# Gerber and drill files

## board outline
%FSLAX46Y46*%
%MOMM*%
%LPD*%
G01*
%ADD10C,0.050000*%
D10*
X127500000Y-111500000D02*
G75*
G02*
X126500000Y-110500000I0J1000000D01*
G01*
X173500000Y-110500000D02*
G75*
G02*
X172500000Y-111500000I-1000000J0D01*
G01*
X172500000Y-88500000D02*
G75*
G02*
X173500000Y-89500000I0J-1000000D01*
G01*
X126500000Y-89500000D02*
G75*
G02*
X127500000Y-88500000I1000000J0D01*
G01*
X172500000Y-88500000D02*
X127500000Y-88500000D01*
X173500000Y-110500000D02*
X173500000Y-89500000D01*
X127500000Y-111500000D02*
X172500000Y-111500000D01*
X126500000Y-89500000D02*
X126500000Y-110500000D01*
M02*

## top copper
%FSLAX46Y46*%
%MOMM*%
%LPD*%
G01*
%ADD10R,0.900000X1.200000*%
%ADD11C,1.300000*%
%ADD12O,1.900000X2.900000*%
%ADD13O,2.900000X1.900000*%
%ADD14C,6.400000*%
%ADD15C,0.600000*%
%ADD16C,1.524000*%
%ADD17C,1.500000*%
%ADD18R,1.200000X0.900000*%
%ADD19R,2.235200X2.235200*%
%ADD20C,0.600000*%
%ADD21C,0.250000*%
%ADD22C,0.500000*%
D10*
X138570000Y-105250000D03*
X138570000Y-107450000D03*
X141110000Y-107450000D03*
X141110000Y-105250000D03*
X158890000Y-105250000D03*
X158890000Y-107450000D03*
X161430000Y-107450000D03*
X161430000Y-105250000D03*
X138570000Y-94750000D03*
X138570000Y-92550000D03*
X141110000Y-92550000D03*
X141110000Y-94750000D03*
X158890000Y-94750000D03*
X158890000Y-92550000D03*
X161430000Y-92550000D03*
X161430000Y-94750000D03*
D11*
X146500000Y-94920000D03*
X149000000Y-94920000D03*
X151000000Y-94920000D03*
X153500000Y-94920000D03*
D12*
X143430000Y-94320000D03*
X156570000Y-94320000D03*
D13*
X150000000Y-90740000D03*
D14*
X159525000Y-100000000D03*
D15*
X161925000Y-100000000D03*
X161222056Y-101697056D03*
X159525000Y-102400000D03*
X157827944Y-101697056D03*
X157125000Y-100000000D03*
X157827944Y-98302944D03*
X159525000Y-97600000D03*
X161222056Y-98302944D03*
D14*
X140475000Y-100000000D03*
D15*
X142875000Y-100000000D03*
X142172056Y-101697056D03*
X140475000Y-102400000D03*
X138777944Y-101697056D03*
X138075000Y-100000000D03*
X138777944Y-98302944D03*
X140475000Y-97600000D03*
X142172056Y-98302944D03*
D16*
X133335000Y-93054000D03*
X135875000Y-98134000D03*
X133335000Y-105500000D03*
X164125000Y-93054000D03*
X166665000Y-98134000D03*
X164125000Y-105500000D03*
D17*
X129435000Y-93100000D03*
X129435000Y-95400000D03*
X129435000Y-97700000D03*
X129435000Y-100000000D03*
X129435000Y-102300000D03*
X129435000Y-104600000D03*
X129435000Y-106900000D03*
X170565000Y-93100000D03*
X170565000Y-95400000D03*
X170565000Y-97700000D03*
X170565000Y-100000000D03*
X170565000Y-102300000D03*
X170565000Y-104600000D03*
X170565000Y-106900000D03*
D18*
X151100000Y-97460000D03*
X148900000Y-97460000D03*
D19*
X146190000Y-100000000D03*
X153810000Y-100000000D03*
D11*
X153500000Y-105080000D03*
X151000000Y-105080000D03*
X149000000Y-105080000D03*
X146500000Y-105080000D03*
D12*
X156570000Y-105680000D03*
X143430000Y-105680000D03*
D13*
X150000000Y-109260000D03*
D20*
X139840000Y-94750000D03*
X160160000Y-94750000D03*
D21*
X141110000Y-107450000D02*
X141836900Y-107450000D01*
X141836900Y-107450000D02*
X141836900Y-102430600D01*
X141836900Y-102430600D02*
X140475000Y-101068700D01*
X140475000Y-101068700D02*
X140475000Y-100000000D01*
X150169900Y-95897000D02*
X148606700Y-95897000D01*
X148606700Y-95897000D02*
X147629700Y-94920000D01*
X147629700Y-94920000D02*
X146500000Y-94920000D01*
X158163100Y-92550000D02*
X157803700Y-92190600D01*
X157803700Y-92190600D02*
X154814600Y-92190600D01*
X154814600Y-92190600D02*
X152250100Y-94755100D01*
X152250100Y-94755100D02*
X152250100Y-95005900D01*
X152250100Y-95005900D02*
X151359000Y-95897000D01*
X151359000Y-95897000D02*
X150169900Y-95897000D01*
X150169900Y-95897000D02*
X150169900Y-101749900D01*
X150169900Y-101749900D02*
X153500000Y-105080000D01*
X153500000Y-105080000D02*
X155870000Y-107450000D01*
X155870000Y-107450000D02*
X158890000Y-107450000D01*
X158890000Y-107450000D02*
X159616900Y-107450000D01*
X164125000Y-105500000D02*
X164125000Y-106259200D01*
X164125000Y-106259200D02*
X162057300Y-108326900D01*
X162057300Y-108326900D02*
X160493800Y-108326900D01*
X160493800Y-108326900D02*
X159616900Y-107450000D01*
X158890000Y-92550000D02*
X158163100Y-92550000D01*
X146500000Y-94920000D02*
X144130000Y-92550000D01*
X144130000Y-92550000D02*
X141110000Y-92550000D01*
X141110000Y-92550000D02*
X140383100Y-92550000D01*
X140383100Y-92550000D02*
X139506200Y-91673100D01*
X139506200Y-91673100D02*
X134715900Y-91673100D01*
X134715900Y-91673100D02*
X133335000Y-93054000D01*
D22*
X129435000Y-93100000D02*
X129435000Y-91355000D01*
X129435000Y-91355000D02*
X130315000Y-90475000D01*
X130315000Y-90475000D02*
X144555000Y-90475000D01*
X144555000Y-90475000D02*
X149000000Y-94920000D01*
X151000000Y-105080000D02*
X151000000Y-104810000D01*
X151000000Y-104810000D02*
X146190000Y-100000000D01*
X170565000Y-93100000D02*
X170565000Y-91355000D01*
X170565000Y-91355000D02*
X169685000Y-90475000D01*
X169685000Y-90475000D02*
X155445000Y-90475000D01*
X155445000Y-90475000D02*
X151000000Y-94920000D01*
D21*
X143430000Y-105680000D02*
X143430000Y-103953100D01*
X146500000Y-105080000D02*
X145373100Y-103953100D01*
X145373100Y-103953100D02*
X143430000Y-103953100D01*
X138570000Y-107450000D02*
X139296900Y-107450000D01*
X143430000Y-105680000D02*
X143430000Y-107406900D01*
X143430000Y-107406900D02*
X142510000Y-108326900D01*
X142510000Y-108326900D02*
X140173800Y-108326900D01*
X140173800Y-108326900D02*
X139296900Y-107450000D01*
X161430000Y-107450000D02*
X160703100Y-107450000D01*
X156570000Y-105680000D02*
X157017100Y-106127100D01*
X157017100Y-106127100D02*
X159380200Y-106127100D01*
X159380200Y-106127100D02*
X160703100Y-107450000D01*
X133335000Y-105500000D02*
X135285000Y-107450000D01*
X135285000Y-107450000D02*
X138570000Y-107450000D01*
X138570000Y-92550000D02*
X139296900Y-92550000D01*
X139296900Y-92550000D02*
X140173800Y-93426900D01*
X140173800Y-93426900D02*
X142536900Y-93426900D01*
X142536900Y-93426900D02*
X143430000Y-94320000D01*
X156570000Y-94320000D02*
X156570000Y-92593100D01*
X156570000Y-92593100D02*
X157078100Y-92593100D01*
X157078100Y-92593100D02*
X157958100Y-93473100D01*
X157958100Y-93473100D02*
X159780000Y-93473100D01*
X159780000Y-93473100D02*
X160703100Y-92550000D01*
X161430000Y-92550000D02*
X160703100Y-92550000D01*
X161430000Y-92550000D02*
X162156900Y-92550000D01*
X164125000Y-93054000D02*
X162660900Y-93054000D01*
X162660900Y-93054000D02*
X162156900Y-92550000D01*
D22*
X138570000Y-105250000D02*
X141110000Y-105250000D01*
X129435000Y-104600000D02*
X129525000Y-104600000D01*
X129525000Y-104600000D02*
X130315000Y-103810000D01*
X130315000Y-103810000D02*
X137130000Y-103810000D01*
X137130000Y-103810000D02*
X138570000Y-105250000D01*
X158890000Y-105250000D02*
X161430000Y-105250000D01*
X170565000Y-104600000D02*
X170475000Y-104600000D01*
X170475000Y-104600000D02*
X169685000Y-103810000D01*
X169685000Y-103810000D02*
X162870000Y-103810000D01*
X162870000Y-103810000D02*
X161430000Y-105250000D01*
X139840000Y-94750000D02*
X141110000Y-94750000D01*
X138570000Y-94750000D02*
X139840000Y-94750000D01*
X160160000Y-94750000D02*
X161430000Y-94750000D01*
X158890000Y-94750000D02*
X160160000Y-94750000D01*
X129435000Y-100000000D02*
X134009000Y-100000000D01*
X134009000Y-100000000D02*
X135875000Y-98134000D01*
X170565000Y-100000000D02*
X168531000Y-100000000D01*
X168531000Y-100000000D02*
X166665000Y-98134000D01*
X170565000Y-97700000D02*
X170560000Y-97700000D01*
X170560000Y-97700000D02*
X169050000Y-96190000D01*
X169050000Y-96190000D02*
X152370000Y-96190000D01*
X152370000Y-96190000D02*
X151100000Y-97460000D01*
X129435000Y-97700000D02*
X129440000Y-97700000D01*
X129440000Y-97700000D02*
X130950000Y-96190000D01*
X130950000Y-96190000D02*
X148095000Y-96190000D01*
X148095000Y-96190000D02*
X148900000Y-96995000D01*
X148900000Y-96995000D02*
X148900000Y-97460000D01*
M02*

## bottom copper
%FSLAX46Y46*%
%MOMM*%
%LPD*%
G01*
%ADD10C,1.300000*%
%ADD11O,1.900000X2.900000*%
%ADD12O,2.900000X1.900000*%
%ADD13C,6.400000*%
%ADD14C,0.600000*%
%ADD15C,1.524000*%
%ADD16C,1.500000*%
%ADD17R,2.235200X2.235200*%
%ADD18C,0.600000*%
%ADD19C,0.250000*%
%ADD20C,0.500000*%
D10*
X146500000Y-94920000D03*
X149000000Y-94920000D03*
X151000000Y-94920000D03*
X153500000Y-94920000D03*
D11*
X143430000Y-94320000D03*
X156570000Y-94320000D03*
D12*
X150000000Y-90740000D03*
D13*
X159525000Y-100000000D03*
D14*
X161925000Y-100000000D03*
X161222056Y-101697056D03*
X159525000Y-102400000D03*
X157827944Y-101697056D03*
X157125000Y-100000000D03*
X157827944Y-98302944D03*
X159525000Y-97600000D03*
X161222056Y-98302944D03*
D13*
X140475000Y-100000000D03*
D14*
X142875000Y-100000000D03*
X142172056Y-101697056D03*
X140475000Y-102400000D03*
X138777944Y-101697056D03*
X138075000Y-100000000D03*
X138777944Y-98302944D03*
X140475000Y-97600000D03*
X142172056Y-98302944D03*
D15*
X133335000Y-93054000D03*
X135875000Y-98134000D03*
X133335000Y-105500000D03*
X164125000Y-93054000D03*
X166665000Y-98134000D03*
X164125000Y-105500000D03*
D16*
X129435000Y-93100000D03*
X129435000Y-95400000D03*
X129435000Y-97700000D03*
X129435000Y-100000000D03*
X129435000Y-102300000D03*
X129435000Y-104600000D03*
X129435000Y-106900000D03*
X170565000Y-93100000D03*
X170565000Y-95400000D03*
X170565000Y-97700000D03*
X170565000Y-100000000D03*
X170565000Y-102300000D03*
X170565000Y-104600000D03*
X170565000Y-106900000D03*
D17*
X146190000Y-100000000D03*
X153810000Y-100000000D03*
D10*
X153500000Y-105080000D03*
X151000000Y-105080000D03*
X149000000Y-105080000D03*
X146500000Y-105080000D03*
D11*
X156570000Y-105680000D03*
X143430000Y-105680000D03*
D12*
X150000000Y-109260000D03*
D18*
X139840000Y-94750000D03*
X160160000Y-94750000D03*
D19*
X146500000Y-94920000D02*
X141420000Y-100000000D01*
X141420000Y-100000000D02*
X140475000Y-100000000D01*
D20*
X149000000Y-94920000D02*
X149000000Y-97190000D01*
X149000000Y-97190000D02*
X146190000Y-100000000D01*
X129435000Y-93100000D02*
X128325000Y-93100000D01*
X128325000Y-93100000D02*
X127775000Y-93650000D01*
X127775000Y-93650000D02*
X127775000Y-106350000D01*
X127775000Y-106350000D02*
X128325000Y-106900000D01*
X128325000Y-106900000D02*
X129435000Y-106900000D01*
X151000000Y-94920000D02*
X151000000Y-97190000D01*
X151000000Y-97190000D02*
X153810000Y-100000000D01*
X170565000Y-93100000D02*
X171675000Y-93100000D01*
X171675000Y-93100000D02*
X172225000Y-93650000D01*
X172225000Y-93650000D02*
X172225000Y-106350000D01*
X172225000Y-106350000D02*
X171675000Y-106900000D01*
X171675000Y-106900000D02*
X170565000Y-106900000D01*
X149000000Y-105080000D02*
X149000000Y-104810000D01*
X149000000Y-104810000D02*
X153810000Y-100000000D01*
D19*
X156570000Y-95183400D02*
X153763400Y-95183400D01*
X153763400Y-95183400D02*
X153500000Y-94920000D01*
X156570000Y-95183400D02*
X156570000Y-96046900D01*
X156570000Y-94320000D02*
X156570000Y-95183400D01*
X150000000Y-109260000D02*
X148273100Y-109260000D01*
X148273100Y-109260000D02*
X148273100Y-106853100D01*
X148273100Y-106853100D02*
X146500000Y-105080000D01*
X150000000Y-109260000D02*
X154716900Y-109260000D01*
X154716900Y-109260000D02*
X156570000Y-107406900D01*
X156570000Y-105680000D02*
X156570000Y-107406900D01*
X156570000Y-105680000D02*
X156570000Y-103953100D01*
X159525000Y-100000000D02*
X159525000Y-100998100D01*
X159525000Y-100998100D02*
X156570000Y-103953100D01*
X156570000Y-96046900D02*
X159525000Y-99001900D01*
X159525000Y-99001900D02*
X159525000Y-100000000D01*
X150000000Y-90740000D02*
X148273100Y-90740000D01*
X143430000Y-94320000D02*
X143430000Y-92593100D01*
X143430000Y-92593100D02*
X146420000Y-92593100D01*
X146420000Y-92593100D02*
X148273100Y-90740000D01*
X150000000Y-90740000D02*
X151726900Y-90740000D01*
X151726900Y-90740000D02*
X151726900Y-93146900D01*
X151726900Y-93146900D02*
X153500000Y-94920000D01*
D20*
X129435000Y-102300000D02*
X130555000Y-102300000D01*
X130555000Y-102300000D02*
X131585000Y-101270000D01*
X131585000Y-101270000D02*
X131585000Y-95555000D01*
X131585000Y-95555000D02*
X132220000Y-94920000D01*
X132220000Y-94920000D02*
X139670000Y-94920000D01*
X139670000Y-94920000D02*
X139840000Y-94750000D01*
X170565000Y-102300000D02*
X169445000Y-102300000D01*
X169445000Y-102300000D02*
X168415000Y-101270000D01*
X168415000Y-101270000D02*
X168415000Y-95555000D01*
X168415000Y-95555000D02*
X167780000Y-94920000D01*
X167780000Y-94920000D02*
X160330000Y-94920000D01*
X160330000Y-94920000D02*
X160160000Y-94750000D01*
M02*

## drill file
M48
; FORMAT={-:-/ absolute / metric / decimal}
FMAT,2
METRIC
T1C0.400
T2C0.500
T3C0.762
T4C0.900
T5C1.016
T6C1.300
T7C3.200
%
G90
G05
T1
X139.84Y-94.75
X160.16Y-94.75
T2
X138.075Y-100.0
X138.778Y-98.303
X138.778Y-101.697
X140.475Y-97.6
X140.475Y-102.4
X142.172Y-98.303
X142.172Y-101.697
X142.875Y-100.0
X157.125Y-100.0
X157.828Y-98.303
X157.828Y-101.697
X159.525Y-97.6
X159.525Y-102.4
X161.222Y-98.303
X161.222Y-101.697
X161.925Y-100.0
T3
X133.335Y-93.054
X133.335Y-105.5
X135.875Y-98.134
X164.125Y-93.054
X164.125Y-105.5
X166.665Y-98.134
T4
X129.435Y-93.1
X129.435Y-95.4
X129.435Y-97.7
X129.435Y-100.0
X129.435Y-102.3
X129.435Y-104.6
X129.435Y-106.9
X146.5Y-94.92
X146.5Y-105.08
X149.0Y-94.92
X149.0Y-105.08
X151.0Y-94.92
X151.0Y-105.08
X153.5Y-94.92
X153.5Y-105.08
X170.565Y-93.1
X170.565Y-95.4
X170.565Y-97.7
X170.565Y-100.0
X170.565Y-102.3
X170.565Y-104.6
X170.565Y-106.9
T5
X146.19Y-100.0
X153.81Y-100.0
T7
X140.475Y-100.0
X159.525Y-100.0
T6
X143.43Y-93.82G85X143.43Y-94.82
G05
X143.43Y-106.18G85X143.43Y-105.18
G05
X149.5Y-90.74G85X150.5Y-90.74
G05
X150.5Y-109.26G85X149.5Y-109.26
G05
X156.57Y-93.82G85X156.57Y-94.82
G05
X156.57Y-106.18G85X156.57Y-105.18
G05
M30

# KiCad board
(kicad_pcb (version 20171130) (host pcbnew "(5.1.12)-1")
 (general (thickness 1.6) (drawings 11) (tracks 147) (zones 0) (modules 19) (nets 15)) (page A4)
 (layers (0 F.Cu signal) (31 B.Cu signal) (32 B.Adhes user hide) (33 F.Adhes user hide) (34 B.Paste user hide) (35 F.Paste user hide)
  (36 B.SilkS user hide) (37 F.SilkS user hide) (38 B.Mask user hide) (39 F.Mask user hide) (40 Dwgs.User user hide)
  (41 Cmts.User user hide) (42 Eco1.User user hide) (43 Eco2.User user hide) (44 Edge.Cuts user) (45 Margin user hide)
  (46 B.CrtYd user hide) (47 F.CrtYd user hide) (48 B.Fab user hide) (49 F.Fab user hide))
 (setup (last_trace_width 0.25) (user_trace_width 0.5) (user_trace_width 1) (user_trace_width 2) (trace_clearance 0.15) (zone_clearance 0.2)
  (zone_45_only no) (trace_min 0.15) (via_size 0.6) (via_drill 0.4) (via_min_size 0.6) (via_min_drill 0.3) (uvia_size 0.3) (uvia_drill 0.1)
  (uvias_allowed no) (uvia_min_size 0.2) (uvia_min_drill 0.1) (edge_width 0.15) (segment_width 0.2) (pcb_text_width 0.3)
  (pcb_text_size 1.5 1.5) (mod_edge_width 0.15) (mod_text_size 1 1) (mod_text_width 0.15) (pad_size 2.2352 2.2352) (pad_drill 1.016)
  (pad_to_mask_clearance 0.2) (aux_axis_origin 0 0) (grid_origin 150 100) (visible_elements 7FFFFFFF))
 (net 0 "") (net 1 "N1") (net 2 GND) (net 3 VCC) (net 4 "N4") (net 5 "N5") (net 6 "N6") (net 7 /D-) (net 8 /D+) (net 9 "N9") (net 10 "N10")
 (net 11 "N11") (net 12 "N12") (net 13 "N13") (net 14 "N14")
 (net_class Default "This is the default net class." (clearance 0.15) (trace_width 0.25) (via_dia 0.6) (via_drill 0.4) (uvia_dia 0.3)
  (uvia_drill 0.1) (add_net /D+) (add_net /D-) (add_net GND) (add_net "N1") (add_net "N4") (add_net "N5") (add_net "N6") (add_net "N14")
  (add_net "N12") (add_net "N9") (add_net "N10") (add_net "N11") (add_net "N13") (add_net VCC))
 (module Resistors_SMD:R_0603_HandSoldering (layer F.Cu) (at 138.57 106.35 270)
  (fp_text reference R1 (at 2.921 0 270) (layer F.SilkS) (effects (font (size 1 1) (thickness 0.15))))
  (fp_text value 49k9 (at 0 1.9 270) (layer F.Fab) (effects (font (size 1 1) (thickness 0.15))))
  (pad 1 smd rect (at -1.1 0 270) (size 1.2 0.9) (layers F.Cu F.Paste F.Mask) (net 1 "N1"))
  (pad 2 smd rect (at 1.1 0 270) (size 1.2 0.9) (layers F.Cu F.Paste F.Mask) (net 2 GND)))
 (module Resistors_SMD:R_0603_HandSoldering (layer F.Cu) (at 141.11 106.35 90)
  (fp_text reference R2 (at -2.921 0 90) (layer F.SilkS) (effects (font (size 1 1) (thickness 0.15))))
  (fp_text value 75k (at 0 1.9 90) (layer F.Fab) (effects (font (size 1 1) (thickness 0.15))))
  (pad 1 smd rect (at -1.1 0 90) (size 1.2 0.9) (layers F.Cu F.Paste F.Mask) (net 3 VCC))
  (pad 2 smd rect (at 1.1 0 90) (size 1.2 0.9) (layers F.Cu F.Paste F.Mask) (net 1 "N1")))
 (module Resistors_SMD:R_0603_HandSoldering (layer F.Cu) (at 158.89 106.35 270)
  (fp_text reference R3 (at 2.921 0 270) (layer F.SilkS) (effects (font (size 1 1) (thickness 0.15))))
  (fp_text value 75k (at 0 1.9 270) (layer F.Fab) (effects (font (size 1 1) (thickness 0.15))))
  (pad 1 smd rect (at -1.1 0 270) (size 1.2 0.9) (layers F.Cu F.Paste F.Mask) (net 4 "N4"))
  (pad 2 smd rect (at 1.1 0 270) (size 1.2 0.9) (layers F.Cu F.Paste F.Mask) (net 3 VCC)))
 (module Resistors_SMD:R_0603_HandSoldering (layer F.Cu) (at 161.43 106.35 90)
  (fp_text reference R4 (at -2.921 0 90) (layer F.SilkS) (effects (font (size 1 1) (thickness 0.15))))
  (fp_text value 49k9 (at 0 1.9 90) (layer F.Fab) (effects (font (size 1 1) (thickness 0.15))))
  (pad 1 smd rect (at -1.1 0 90) (size 1.2 0.9) (layers F.Cu F.Paste F.Mask) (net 2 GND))
  (pad 2 smd rect (at 1.1 0 90) (size 1.2 0.9) (layers F.Cu F.Paste F.Mask) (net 4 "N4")))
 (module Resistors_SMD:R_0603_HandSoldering (layer F.Cu) (at 138.57 93.65 90)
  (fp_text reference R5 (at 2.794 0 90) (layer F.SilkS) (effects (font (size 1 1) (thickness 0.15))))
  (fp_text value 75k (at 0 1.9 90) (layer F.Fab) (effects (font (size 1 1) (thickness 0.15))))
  (pad 1 smd rect (at -1.1 0 90) (size 1.2 0.9) (layers F.Cu F.Paste F.Mask) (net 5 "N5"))
  (pad 2 smd rect (at 1.1 0 90) (size 1.2 0.9) (layers F.Cu F.Paste F.Mask) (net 2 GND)))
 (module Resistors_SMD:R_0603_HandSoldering (layer F.Cu) (at 141.11 93.65 270)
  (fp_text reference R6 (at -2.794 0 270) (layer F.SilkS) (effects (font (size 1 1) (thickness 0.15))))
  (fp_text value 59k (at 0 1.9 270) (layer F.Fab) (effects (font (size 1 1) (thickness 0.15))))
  (pad 1 smd rect (at -1.1 0 270) (size 1.2 0.9) (layers F.Cu F.Paste F.Mask) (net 3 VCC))
  (pad 2 smd rect (at 1.1 0 270) (size 1.2 0.9) (layers F.Cu F.Paste F.Mask) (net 5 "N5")))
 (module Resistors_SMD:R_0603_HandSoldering (layer F.Cu) (at 158.89 93.65 90)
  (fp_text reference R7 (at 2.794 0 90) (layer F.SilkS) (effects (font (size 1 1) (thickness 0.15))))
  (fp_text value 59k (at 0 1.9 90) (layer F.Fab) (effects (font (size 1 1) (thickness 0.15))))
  (pad 1 smd rect (at -1.1 0 90) (size 1.2 0.9) (layers F.Cu F.Paste F.Mask) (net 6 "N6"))
  (pad 2 smd rect (at 1.1 0 90) (size 1.2 0.9) (layers F.Cu F.Paste F.Mask) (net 3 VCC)))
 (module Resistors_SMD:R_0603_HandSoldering (layer F.Cu) (at 161.43 93.65 270)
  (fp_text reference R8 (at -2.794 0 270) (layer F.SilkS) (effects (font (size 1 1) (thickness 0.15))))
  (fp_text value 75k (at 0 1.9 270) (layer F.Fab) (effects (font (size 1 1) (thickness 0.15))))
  (pad 1 smd rect (at -1.1 0 270) (size 1.2 0.9) (layers F.Cu F.Paste F.Mask) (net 2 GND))
  (pad 2 smd rect (at 1.1 0 270) (size 1.2 0.9) (layers F.Cu F.Paste F.Mask) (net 6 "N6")))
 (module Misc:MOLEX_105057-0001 (layer F.Cu) (at 150 94.92)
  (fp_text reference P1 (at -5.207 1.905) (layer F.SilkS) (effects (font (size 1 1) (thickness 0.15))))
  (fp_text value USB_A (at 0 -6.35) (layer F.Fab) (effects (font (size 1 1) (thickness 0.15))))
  (pad 1 thru_hole circle (at -3.5 0) (size 1.3 1.3) (drill 0.9) (layers *.Cu *.Mask) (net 3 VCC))
  (pad 2 thru_hole circle (at -1 0) (size 1.3 1.3) (drill 0.9) (layers *.Cu *.Mask) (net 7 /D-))
  (pad 3 thru_hole circle (at 1 0) (size 1.3 1.3) (drill 0.9) (layers *.Cu *.Mask) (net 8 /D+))
  (pad 4 thru_hole circle (at 3.5 0) (size 1.3 1.3) (drill 0.9) (layers *.Cu *.Mask) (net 2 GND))
  (pad 5 thru_hole oval (at -6.57 -0.6) (size 1.9 2.9) (drill oval 1.3 2.3) (layers *.Cu *.Mask) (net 2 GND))
  (pad 5 thru_hole oval (at 6.57 -0.6) (size 1.9 2.9) (drill oval 1.3 2.3) (layers *.Cu *.Mask) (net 2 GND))
  (pad 5 thru_hole oval (at 0 -4.18) (size 2.9 1.9) (drill oval 2.3 1.3) (layers *.Cu *.Mask) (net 2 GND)))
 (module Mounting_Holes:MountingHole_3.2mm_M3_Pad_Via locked (layer F.Cu) (at 159.525 100)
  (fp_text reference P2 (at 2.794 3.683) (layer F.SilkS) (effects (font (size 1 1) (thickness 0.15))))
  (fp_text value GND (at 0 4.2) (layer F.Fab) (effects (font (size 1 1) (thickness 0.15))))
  (pad 1 thru_hole circle (at 0 0) (size 6.4 6.4) (drill 3.2) (layers *.Cu *.Mask F.SilkS) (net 2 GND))
  (pad "" thru_hole circle (at 2.4 0) (size 0.6 0.6) (drill 0.5) (layers *.Cu *.Mask))
  (pad "" thru_hole circle (at 1.697056 1.697056) (size 0.6 0.6) (drill 0.5) (layers *.Cu *.Mask))
  (pad "" thru_hole circle (at 0 2.4) (size 0.6 0.6) (drill 0.5) (layers *.Cu *.Mask))
  (pad "" thru_hole circle (at -1.697056 1.697056) (size 0.6 0.6) (drill 0.5) (layers *.Cu *.Mask))
  (pad "" thru_hole circle (at -2.4 0) (size 0.6 0.6) (drill 0.5) (layers *.Cu *.Mask))
  (pad "" thru_hole circle (at -1.697056 -1.697056) (size 0.6 0.6) (drill 0.5) (layers *.Cu *.Mask))
  (pad "" thru_hole circle (at 0 -2.4) (size 0.6 0.6) (drill 0.5) (layers *.Cu *.Mask))
  (pad "" thru_hole circle (at 1.697056 -1.697056) (size 0.6 0.6) (drill 0.5) (layers *.Cu *.Mask)))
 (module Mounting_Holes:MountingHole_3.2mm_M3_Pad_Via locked (layer F.Cu) (at 140.475 100)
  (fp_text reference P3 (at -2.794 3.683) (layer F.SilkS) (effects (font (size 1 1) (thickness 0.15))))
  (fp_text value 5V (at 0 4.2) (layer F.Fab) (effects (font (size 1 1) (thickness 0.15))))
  (pad 1 thru_hole circle (at 0 0) (size 6.4 6.4) (drill 3.2) (layers *.Cu *.Mask F.SilkS) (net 3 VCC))
  (pad "" thru_hole circle (at 2.4 0) (size 0.6 0.6) (drill 0.5) (layers *.Cu *.Mask))
  (pad "" thru_hole circle (at 1.697056 1.697056) (size 0.6 0.6) (drill 0.5) (layers *.Cu *.Mask))
  (pad "" thru_hole circle (at 0 2.4) (size 0.6 0.6) (drill 0.5) (layers *.Cu *.Mask))
  (pad "" thru_hole circle (at -1.697056 1.697056) (size 0.6 0.6) (drill 0.5) (layers *.Cu *.Mask))
  (pad "" thru_hole circle (at -2.4 0) (size 0.6 0.6) (drill 0.5) (layers *.Cu *.Mask))
  (pad "" thru_hole circle (at -1.697056 -1.697056) (size 0.6 0.6) (drill 0.5) (layers *.Cu *.Mask))
  (pad "" thru_hole circle (at 0 -2.4) (size 0.6 0.6) (drill 0.5) (layers *.Cu *.Mask))
  (pad "" thru_hole circle (at 1.697056 -1.697056) (size 0.6 0.6) (drill 0.5) (layers *.Cu *.Mask)))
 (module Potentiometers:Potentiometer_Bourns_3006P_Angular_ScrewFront (layer F.Cu) (at 133.335 105.5 270)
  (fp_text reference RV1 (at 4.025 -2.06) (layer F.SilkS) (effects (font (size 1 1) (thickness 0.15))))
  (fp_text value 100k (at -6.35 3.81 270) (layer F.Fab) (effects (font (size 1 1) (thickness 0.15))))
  (pad 3 thru_hole circle (at -12.446 0 270) (size 1.524 1.524) (drill 0.762) (layers *.Cu *.Mask F.SilkS) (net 3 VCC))
  (pad 2 thru_hole circle (at -7.366 -2.54 270) (size 1.524 1.524) (drill 0.762) (layers *.Cu *.Mask F.SilkS) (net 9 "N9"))
  (pad 1 thru_hole circle (at 0 0 270) (size 1.524 1.524) (drill 0.762) (layers *.Cu *.Mask F.SilkS) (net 2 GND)))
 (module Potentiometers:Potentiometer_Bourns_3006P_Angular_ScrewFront (layer F.Cu) (at 164.125 105.5 270)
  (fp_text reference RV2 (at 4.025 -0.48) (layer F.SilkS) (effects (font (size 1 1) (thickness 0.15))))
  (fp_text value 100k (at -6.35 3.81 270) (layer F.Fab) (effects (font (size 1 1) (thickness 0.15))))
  (pad 3 thru_hole circle (at -12.446 0 270) (size 1.524 1.524) (drill 0.762) (layers *.Cu *.Mask F.SilkS) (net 2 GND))
  (pad 2 thru_hole circle (at -7.366 -2.54 270) (size 1.524 1.524) (drill 0.762) (layers *.Cu *.Mask F.SilkS) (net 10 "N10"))
  (pad 1 thru_hole circle (at 0 0 270) (size 1.524 1.524) (drill 0.762) (layers *.Cu *.Mask F.SilkS) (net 3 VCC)))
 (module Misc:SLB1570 (layer F.Cu) (at 129.435 100 270)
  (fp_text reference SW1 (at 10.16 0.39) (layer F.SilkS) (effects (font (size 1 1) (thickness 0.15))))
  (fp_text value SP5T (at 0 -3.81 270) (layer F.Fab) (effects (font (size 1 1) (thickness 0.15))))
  (pad C thru_hole circle (at -6.9 0 270) (size 1.5 1.5) (drill 0.9) (layers *.Cu *.Mask F.SilkS) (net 7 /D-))
  (pad 1 thru_hole circle (at -4.6 0 270) (size 1.5 1.5) (drill 0.9) (layers *.Cu *.Mask F.SilkS) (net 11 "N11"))
  (pad 2 thru_hole circle (at -2.3 0 270) (size 1.5 1.5) (drill 0.9) (layers *.Cu *.Mask F.SilkS) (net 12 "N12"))
  (pad 3 thru_hole circle (at 0 0 270) (size 1.5 1.5) (drill 0.9) (layers *.Cu *.Mask F.SilkS) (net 9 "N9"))
  (pad 4 thru_hole circle (at 2.3 0 270) (size 1.5 1.5) (drill 0.9) (layers *.Cu *.Mask F.SilkS) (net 5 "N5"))
  (pad 5 thru_hole circle (at 4.6 0 270) (size 1.5 1.5) (drill 0.9) (layers *.Cu *.Mask F.SilkS) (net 1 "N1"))
  (pad C thru_hole circle (at 6.9 0 270) (size 1.5 1.5) (drill 0.9) (layers *.Cu *.Mask F.SilkS) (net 7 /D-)))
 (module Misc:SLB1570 (layer F.Cu) (at 170.565 100 270)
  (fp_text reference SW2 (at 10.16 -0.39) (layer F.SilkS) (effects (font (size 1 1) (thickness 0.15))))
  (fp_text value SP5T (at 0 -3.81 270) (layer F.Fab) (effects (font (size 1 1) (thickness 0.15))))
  (pad C thru_hole circle (at -6.9 0 270) (size 1.5 1.5) (drill 0.9) (layers *.Cu *.Mask F.SilkS) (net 8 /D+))
  (pad 1 thru_hole circle (at -4.6 0 270) (size 1.5 1.5) (drill 0.9) (layers *.Cu *.Mask F.SilkS) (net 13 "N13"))
  (pad 2 thru_hole circle (at -2.3 0 270) (size 1.5 1.5) (drill 0.9) (layers *.Cu *.Mask F.SilkS) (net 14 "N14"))
  (pad 3 thru_hole circle (at 0 0 270) (size 1.5 1.5) (drill 0.9) (layers *.Cu *.Mask F.SilkS) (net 10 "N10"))
  (pad 4 thru_hole circle (at 2.3 0 270) (size 1.5 1.5) (drill 0.9) (layers *.Cu *.Mask F.SilkS) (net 6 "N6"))
  (pad 5 thru_hole circle (at 4.6 0 270) (size 1.5 1.5) (drill 0.9) (layers *.Cu *.Mask F.SilkS) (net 4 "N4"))
  (pad C thru_hole circle (at 6.9 0 270) (size 1.5 1.5) (drill 0.9) (layers *.Cu *.Mask F.SilkS) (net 8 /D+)))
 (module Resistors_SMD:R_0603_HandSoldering (layer F.Cu) (at 150 97.46 180)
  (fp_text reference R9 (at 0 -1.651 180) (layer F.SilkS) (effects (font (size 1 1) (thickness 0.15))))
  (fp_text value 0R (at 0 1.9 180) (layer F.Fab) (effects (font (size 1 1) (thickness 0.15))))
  (pad 1 smd rect (at -1.1 0 180) (size 1.2 0.9) (layers F.Cu F.Paste F.Mask) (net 14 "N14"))
  (pad 2 smd rect (at 1.1 0 180) (size 1.2 0.9) (layers F.Cu F.Paste F.Mask) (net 12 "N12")))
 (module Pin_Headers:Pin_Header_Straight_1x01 (layer F.Cu) (at 146.19 100)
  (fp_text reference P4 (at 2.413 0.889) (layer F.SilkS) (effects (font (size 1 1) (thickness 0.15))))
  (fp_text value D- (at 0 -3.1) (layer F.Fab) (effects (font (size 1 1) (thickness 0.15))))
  (pad 1 thru_hole rect (at 0 0) (size 2.2352 2.2352) (drill 1.016) (layers *.Cu *.Mask F.SilkS) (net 7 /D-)))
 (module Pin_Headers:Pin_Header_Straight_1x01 (layer F.Cu) (at 153.81 100)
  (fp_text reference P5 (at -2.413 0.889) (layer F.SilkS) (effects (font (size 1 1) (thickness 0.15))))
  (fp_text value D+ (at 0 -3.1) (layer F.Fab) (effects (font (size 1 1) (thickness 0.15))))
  (pad 1 thru_hole rect (at 0 0) (size 2.2352 2.2352) (drill 1.016) (layers *.Cu *.Mask F.SilkS) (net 8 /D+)))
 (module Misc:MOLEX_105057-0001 (layer F.Cu) (at 150 105.08 180)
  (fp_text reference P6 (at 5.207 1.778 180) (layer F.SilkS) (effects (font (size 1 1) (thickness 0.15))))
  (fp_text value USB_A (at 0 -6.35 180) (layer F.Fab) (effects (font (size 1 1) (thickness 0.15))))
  (pad 1 thru_hole circle (at -3.5 0 180) (size 1.3 1.3) (drill 0.9) (layers *.Cu *.Mask) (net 3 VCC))
  (pad 2 thru_hole circle (at -1 0 180) (size 1.3 1.3) (drill 0.9) (layers *.Cu *.Mask) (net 7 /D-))
  (pad 3 thru_hole circle (at 1 0 180) (size 1.3 1.3) (drill 0.9) (layers *.Cu *.Mask) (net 8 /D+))
  (pad 4 thru_hole circle (at 3.5 0 180) (size 1.3 1.3) (drill 0.9) (layers *.Cu *.Mask) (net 2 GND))
  (pad 5 thru_hole oval (at -6.57 -0.6 180) (size 1.9 2.9) (drill oval 1.3 2.3) (layers *.Cu *.Mask) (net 2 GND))
  (pad 5 thru_hole oval (at 6.57 -0.6 180) (size 1.9 2.9) (drill oval 1.3 2.3) (layers *.Cu *.Mask) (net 2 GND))
  (pad 5 thru_hole oval (at 0 -4.18 180) (size 2.9 1.9) (drill oval 2.3 1.3) (layers *.Cu *.Mask) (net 2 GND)))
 (gr_arc (start 127.5 110.5) (end 127.5 111.5) (angle 90) (layer Edge.Cuts) (width 0.05))
 (gr_arc (start 172.5 110.5) (end 173.5 110.5) (angle 90) (layer Edge.Cuts) (width 0.05))
 (gr_arc (start 172.5 89.5) (end 172.5 88.5) (angle 90) (layer Edge.Cuts) (width 0.05))
 (gr_arc (start 127.5 89.5) (end 126.5 89.5) (angle 90) (layer Edge.Cuts) (width 0.05))
 (gr_line (start 172.5 88.5) (end 127.5 88.5) (angle 90) (layer Edge.Cuts) (width 0.05))
 (gr_line (start 173.5 110.5) (end 173.5 89.5) (angle 90) (layer Edge.Cuts) (width 0.05))
 (gr_line (start 127.5 111.5) (end 172.5 111.5) (angle 90) (layer Edge.Cuts) (width 0.05))
 (gr_line (start 126.5 89.5) (end 126.5 110.5) (angle 90) (layer Edge.Cuts) (width 0.05))
 (segment (start 141.11 107.45) (end 141.8369 107.45) (width 0.25) (layer F.Cu) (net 3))
 (segment (start 141.8369 107.45) (end 141.8369 102.4306) (width 0.25) (layer F.Cu) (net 3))
 (segment (start 141.8369 102.4306) (end 140.475 101.0687) (width 0.25) (layer F.Cu) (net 3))
 (segment (start 140.475 101.0687) (end 140.475 100) (width 0.25) (layer F.Cu) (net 3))
 (segment (start 150.1699 95.897) (end 148.6067 95.897) (width 0.25) (layer F.Cu) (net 3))
 (segment (start 148.6067 95.897) (end 147.6297 94.92) (width 0.25) (layer F.Cu) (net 3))
 (segment (start 147.6297 94.92) (end 146.5 94.92) (width 0.25) (layer F.Cu) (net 3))
 (segment (start 158.1631 92.55) (end 157.8037 92.1906) (width 0.25) (layer F.Cu) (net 3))
 (segment (start 157.8037 92.1906) (end 154.8146 92.1906) (width 0.25) (layer F.Cu) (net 3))
 (segment (start 154.8146 92.1906) (end 152.2501 94.7551) (width 0.25) (layer F.Cu) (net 3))
 (segment (start 152.2501 94.7551) (end 152.2501 95.0059) (width 0.25) (layer F.Cu) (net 3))
 (segment (start 152.2501 95.0059) (end 151.359 95.897) (width 0.25) (layer F.Cu) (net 3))
 (segment (start 151.359 95.897) (end 150.1699 95.897) (width 0.25) (layer F.Cu) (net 3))
 (segment (start 150.1699 95.897) (end 150.1699 101.7499) (width 0.25) (layer F.Cu) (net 3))
 (segment (start 150.1699 101.7499) (end 153.5 105.08) (width 0.25) (layer F.Cu) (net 3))
 (segment (start 153.5 105.08) (end 155.87 107.45) (width 0.25) (layer F.Cu) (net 3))
 (segment (start 155.87 107.45) (end 158.89 107.45) (width 0.25) (layer F.Cu) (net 3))
 (segment (start 158.89 107.45) (end 159.6169 107.45) (width 0.25) (layer F.Cu) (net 3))
 (segment (start 164.125 105.5) (end 164.125 106.2592) (width 0.25) (layer F.Cu) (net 3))
 (segment (start 164.125 106.2592) (end 162.0573 108.3269) (width 0.25) (layer F.Cu) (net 3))
 (segment (start 162.0573 108.3269) (end 160.4938 108.3269) (width 0.25) (layer F.Cu) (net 3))
 (segment (start 160.4938 108.3269) (end 159.6169 107.45) (width 0.25) (layer F.Cu) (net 3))
 (segment (start 158.89 92.55) (end 158.1631 92.55) (width 0.25) (layer F.Cu) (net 3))
 (segment (start 146.5 94.92) (end 144.13 92.55) (width 0.25) (layer F.Cu) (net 3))
 (segment (start 144.13 92.55) (end 141.11 92.55) (width 0.25) (layer F.Cu) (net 3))
 (segment (start 146.5 94.92) (end 141.42 100) (width 0.25) (layer B.Cu) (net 3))
 (segment (start 141.42 100) (end 140.475 100) (width 0.25) (layer B.Cu) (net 3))
 (segment (start 141.11 92.55) (end 140.3831 92.55) (width 0.25) (layer F.Cu) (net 3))
 (segment (start 140.3831 92.55) (end 139.5062 91.6731) (width 0.25) (layer F.Cu) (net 3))
 (segment (start 139.5062 91.6731) (end 134.7159 91.6731) (width 0.25) (layer F.Cu) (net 3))
 (segment (start 134.7159 91.6731) (end 133.335 93.054) (width 0.25) (layer F.Cu) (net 3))
 (segment (start 129.435 93.1) (end 129.435 91.355) (width 0.5) (layer F.Cu) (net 7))
 (segment (start 129.435 91.355) (end 130.315 90.475) (width 0.5) (layer F.Cu) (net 7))
 (segment (start 130.315 90.475) (end 144.555 90.475) (width 0.5) (layer F.Cu) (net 7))
 (segment (start 144.555 90.475) (end 149 94.92) (width 0.5) (layer F.Cu) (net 7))
 (segment (start 149 94.92) (end 149 97.19) (width 0.5) (layer B.Cu) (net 7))
 (segment (start 149 97.19) (end 146.19 100) (width 0.5) (layer B.Cu) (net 7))
 (segment (start 129.435 93.1) (end 128.325 93.1) (width 0.5) (layer B.Cu) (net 7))
 (segment (start 128.325 93.1) (end 127.775 93.65) (width 0.5) (layer B.Cu) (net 7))
 (segment (start 127.775 93.65) (end 127.775 106.35) (width 0.5) (layer B.Cu) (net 7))
 (segment (start 127.775 106.35) (end 128.325 106.9) (width 0.5) (layer B.Cu) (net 7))
 (segment (start 128.325 106.9) (end 129.435 106.9) (width 0.5) (layer B.Cu) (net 7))
 (segment (start 151 105.08) (end 151 104.81) (width 0.5) (layer F.Cu) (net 7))
 (segment (start 151 104.81) (end 146.19 100) (width 0.5) (layer F.Cu) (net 7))
 (segment (start 170.565 93.1) (end 170.565 91.355) (width 0.5) (layer F.Cu) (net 8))
 (segment (start 170.565 91.355) (end 169.685 90.475) (width 0.5) (layer F.Cu) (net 8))
 (segment (start 169.685 90.475) (end 155.445 90.475) (width 0.5) (layer F.Cu) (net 8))
 (segment (start 155.445 90.475) (end 151 94.92) (width 0.5) (layer F.Cu) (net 8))
 (segment (start 151 94.92) (end 151 97.19) (width 0.5) (layer B.Cu) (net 8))
 (segment (start 151 97.19) (end 153.81 100) (width 0.5) (layer B.Cu) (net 8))
 (segment (start 170.565 93.1) (end 171.675 93.1) (width 0.5) (layer B.Cu) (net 8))
 (segment (start 171.675 93.1) (end 172.225 93.65) (width 0.5) (layer B.Cu) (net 8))
 (segment (start 172.225 93.65) (end 172.225 106.35) (width 0.5) (layer B.Cu) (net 8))
 (segment (start 172.225 106.35) (end 171.675 106.9) (width 0.5) (layer B.Cu) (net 8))
 (segment (start 171.675 106.9) (end 170.565 106.9) (width 0.5) (layer B.Cu) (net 8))
 (segment (start 149 105.08) (end 149 104.81) (width 0.5) (layer B.Cu) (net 8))
 (segment (start 149 104.81) (end 153.81 100) (width 0.5) (layer B.Cu) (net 8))
 (segment (start 143.43 105.68) (end 143.43 103.9531) (width 0.25) (layer F.Cu) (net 2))
 (segment (start 146.5 105.08) (end 145.3731 103.9531) (width 0.25) (layer F.Cu) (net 2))
 (segment (start 145.3731 103.9531) (end 143.43 103.9531) (width 0.25) (layer F.Cu) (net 2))
 (segment (start 138.57 107.45) (end 139.2969 107.45) (width 0.25) (layer F.Cu) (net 2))
 (segment (start 143.43 105.68) (end 143.43 107.4069) (width 0.25) (layer F.Cu) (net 2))
 (segment (start 143.43 107.4069) (end 142.51 108.3269) (width 0.25) (layer F.Cu) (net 2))
 (segment (start 142.51 108.3269) (end 140.1738 108.3269) (width 0.25) (layer F.Cu) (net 2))
 (segment (start 140.1738 108.3269) (end 139.2969 107.45) (width 0.25) (layer F.Cu) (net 2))
 (segment (start 161.43 107.45) (end 160.7031 107.45) (width 0.25) (layer F.Cu) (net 2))
 (segment (start 156.57 105.68) (end 157.0171 106.1271) (width 0.25) (layer F.Cu) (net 2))
 (segment (start 157.0171 106.1271) (end 159.3802 106.1271) (width 0.25) (layer F.Cu) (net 2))
 (segment (start 159.3802 106.1271) (end 160.7031 107.45) (width 0.25) (layer F.Cu) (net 2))
 (segment (start 156.57 95.1834) (end 153.7634 95.1834) (width 0.25) (layer B.Cu) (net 2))
 (segment (start 153.7634 95.1834) (end 153.5 94.92) (width 0.25) (layer B.Cu) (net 2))
 (segment (start 156.57 95.1834) (end 156.57 96.0469) (width 0.25) (layer B.Cu) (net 2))
 (segment (start 156.57 94.32) (end 156.57 95.1834) (width 0.25) (layer B.Cu) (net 2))
 (segment (start 150 109.26) (end 148.2731 109.26) (width 0.25) (layer B.Cu) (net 2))
 (segment (start 148.2731 109.26) (end 148.2731 106.8531) (width 0.25) (layer B.Cu) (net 2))
 (segment (start 148.2731 106.8531) (end 146.5 105.08) (width 0.25) (layer B.Cu) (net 2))
 (segment (start 150 109.26) (end 154.7169 109.26) (width 0.25) (layer B.Cu) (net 2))
 (segment (start 154.7169 109.26) (end 156.57 107.4069) (width 0.25) (layer B.Cu) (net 2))
 (segment (start 156.57 105.68) (end 156.57 107.4069) (width 0.25) (layer B.Cu) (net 2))
 (segment (start 156.57 105.68) (end 156.57 103.9531) (width 0.25) (layer B.Cu) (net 2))
 (segment (start 159.525 100) (end 159.525 100.9981) (width 0.25) (layer B.Cu) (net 2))
 (segment (start 159.525 100.9981) (end 156.57 103.9531) (width 0.25) (layer B.Cu) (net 2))
 (segment (start 156.57 96.0469) (end 159.525 99.0019) (width 0.25) (layer B.Cu) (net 2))
 (segment (start 159.525 99.0019) (end 159.525 100) (width 0.25) (layer B.Cu) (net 2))
 (segment (start 133.335 105.5) (end 135.285 107.45) (width 0.25) (layer F.Cu) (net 2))
 (segment (start 135.285 107.45) (end 138.57 107.45) (width 0.25) (layer F.Cu) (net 2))
 (segment (start 138.57 92.55) (end 139.2969 92.55) (width 0.25) (layer F.Cu) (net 2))
 (segment (start 139.2969 92.55) (end 140.1738 93.4269) (width 0.25) (layer F.Cu) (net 2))
 (segment (start 140.1738 93.4269) (end 142.5369 93.4269) (width 0.25) (layer F.Cu) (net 2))
 (segment (start 142.5369 93.4269) (end 143.43 94.32) (width 0.25) (layer F.Cu) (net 2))
 (segment (start 156.57 94.32) (end 156.57 92.5931) (width 0.25) (layer F.Cu) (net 2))
 (segment (start 156.57 92.5931) (end 157.0781 92.5931) (width 0.25) (layer F.Cu) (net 2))
 (segment (start 157.0781 92.5931) (end 157.9581 93.4731) (width 0.25) (layer F.Cu) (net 2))
 (segment (start 157.9581 93.4731) (end 159.78 93.4731) (width 0.25) (layer F.Cu) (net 2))
 (segment (start 159.78 93.4731) (end 160.7031 92.55) (width 0.25) (layer F.Cu) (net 2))
 (segment (start 161.43 92.55) (end 160.7031 92.55) (width 0.25) (layer F.Cu) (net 2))
 (segment (start 150 90.74) (end 148.2731 90.74) (width 0.25) (layer B.Cu) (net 2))
 (segment (start 143.43 94.32) (end 143.43 92.5931) (width 0.25) (layer B.Cu) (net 2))
 (segment (start 143.43 92.5931) (end 146.42 92.5931) (width 0.25) (layer B.Cu) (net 2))
 (segment (start 146.42 92.5931) (end 148.2731 90.74) (width 0.25) (layer B.Cu) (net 2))
 (segment (start 150 90.74) (end 151.7269 90.74) (width 0.25) (layer B.Cu) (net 2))
 (segment (start 151.7269 90.74) (end 151.7269 93.1469) (width 0.25) (layer B.Cu) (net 2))
 (segment (start 151.7269 93.1469) (end 153.5 94.92) (width 0.25) (layer B.Cu) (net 2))
 (segment (start 161.43 92.55) (end 162.1569 92.55) (width 0.25) (layer F.Cu) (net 2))
 (segment (start 164.125 93.054) (end 162.6609 93.054) (width 0.25) (layer F.Cu) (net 2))
 (segment (start 162.6609 93.054) (end 162.1569 92.55) (width 0.25) (layer F.Cu) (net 2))
 (segment (start 138.57 105.25) (end 141.11 105.25) (width 0.5) (layer F.Cu) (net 1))
 (segment (start 129.435 104.6) (end 129.525 104.6) (width 0.5) (layer F.Cu) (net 1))
 (segment (start 129.525 104.6) (end 130.315 103.81) (width 0.5) (layer F.Cu) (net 1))
 (segment (start 130.315 103.81) (end 137.13 103.81) (width 0.5) (layer F.Cu) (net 1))
 (segment (start 137.13 103.81) (end 138.57 105.25) (width 0.5) (layer F.Cu) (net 1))
 (segment (start 158.89 105.25) (end 161.43 105.25) (width 0.5) (layer F.Cu) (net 4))
 (segment (start 170.565 104.6) (end 170.475 104.6) (width 0.5) (layer F.Cu) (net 4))
 (segment (start 170.475 104.6) (end 169.685 103.81) (width 0.5) (layer F.Cu) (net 4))
 (segment (start 169.685 103.81) (end 162.87 103.81) (width 0.5) (layer F.Cu) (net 4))
 (segment (start 162.87 103.81) (end 161.43 105.25) (width 0.5) (layer F.Cu) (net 4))
 (segment (start 139.84 94.75) (end 141.11 94.75) (width 0.5) (layer F.Cu) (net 5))
 (segment (start 138.57 94.75) (end 139.84 94.75) (width 0.5) (layer F.Cu) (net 5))
 (segment (start 129.435 102.3) (end 130.555 102.3) (width 0.5) (layer B.Cu) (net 5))
 (segment (start 130.555 102.3) (end 131.585 101.27) (width 0.5) (layer B.Cu) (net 5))
 (segment (start 131.585 101.27) (end 131.585 95.555) (width 0.5) (layer B.Cu) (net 5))
 (segment (start 131.585 95.555) (end 132.22 94.92) (width 0.5) (layer B.Cu) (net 5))
 (segment (start 132.22 94.92) (end 139.67 94.92) (width 0.5) (layer B.Cu) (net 5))
 (segment (start 139.67 94.92) (end 139.84 94.75) (width 0.5) (layer B.Cu) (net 5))
 (via (at 139.84 94.75) (size 0.6) (layers F.Cu B.Cu) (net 5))
 (segment (start 160.16 94.75) (end 161.43 94.75) (width 0.5) (layer F.Cu) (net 6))
 (segment (start 158.89 94.75) (end 160.16 94.75) (width 0.5) (layer F.Cu) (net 6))
 (segment (start 170.565 102.3) (end 169.445 102.3) (width 0.5) (layer B.Cu) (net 6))
 (segment (start 169.445 102.3) (end 168.415 101.27) (width 0.5) (layer B.Cu) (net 6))
 (segment (start 168.415 101.27) (end 168.415 95.555) (width 0.5) (layer B.Cu) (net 6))
 (segment (start 168.415 95.555) (end 167.78 94.92) (width 0.5) (layer B.Cu) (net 6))
 (segment (start 167.78 94.92) (end 160.33 94.92) (width 0.5) (layer B.Cu) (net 6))
 (segment (start 160.33 94.92) (end 160.16 94.75) (width 0.5) (layer B.Cu) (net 6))
 (via (at 160.16 94.75) (size 0.6) (layers F.Cu B.Cu) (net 6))
 (segment (start 129.435 100) (end 134.009 100) (width 0.5) (layer F.Cu) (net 9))
 (segment (start 134.009 100) (end 135.875 98.134) (width 0.5) (layer F.Cu) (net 9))
 (segment (start 170.565 100) (end 168.531 100) (width 0.5) (layer F.Cu) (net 10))
 (segment (start 168.531 100) (end 166.665 98.134) (width 0.5) (layer F.Cu) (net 10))
 (segment (start 170.565 97.7) (end 170.56 97.7) (width 0.5) (layer F.Cu) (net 14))
 (segment (start 170.56 97.7) (end 169.05 96.19) (width 0.5) (layer F.Cu) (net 14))
 (segment (start 169.05 96.19) (end 152.37 96.19) (width 0.5) (layer F.Cu) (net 14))
 (segment (start 152.37 96.19) (end 151.1 97.46) (width 0.5) (layer F.Cu) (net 14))
 (segment (start 129.435 97.7) (end 129.44 97.7) (width 0.5) (layer F.Cu) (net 12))
 (segment (start 129.44 97.7) (end 130.95 96.19) (width 0.5) (layer F.Cu) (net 12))
 (segment (start 130.95 96.19) (end 148.095 96.19) (width 0.5) (layer F.Cu) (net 12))
 (segment (start 148.095 96.19) (end 148.9 96.995) (width 0.5) (layer F.Cu) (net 12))
 (segment (start 148.9 96.995) (end 148.9 97.46) (width 0.5) (layer F.Cu) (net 12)))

